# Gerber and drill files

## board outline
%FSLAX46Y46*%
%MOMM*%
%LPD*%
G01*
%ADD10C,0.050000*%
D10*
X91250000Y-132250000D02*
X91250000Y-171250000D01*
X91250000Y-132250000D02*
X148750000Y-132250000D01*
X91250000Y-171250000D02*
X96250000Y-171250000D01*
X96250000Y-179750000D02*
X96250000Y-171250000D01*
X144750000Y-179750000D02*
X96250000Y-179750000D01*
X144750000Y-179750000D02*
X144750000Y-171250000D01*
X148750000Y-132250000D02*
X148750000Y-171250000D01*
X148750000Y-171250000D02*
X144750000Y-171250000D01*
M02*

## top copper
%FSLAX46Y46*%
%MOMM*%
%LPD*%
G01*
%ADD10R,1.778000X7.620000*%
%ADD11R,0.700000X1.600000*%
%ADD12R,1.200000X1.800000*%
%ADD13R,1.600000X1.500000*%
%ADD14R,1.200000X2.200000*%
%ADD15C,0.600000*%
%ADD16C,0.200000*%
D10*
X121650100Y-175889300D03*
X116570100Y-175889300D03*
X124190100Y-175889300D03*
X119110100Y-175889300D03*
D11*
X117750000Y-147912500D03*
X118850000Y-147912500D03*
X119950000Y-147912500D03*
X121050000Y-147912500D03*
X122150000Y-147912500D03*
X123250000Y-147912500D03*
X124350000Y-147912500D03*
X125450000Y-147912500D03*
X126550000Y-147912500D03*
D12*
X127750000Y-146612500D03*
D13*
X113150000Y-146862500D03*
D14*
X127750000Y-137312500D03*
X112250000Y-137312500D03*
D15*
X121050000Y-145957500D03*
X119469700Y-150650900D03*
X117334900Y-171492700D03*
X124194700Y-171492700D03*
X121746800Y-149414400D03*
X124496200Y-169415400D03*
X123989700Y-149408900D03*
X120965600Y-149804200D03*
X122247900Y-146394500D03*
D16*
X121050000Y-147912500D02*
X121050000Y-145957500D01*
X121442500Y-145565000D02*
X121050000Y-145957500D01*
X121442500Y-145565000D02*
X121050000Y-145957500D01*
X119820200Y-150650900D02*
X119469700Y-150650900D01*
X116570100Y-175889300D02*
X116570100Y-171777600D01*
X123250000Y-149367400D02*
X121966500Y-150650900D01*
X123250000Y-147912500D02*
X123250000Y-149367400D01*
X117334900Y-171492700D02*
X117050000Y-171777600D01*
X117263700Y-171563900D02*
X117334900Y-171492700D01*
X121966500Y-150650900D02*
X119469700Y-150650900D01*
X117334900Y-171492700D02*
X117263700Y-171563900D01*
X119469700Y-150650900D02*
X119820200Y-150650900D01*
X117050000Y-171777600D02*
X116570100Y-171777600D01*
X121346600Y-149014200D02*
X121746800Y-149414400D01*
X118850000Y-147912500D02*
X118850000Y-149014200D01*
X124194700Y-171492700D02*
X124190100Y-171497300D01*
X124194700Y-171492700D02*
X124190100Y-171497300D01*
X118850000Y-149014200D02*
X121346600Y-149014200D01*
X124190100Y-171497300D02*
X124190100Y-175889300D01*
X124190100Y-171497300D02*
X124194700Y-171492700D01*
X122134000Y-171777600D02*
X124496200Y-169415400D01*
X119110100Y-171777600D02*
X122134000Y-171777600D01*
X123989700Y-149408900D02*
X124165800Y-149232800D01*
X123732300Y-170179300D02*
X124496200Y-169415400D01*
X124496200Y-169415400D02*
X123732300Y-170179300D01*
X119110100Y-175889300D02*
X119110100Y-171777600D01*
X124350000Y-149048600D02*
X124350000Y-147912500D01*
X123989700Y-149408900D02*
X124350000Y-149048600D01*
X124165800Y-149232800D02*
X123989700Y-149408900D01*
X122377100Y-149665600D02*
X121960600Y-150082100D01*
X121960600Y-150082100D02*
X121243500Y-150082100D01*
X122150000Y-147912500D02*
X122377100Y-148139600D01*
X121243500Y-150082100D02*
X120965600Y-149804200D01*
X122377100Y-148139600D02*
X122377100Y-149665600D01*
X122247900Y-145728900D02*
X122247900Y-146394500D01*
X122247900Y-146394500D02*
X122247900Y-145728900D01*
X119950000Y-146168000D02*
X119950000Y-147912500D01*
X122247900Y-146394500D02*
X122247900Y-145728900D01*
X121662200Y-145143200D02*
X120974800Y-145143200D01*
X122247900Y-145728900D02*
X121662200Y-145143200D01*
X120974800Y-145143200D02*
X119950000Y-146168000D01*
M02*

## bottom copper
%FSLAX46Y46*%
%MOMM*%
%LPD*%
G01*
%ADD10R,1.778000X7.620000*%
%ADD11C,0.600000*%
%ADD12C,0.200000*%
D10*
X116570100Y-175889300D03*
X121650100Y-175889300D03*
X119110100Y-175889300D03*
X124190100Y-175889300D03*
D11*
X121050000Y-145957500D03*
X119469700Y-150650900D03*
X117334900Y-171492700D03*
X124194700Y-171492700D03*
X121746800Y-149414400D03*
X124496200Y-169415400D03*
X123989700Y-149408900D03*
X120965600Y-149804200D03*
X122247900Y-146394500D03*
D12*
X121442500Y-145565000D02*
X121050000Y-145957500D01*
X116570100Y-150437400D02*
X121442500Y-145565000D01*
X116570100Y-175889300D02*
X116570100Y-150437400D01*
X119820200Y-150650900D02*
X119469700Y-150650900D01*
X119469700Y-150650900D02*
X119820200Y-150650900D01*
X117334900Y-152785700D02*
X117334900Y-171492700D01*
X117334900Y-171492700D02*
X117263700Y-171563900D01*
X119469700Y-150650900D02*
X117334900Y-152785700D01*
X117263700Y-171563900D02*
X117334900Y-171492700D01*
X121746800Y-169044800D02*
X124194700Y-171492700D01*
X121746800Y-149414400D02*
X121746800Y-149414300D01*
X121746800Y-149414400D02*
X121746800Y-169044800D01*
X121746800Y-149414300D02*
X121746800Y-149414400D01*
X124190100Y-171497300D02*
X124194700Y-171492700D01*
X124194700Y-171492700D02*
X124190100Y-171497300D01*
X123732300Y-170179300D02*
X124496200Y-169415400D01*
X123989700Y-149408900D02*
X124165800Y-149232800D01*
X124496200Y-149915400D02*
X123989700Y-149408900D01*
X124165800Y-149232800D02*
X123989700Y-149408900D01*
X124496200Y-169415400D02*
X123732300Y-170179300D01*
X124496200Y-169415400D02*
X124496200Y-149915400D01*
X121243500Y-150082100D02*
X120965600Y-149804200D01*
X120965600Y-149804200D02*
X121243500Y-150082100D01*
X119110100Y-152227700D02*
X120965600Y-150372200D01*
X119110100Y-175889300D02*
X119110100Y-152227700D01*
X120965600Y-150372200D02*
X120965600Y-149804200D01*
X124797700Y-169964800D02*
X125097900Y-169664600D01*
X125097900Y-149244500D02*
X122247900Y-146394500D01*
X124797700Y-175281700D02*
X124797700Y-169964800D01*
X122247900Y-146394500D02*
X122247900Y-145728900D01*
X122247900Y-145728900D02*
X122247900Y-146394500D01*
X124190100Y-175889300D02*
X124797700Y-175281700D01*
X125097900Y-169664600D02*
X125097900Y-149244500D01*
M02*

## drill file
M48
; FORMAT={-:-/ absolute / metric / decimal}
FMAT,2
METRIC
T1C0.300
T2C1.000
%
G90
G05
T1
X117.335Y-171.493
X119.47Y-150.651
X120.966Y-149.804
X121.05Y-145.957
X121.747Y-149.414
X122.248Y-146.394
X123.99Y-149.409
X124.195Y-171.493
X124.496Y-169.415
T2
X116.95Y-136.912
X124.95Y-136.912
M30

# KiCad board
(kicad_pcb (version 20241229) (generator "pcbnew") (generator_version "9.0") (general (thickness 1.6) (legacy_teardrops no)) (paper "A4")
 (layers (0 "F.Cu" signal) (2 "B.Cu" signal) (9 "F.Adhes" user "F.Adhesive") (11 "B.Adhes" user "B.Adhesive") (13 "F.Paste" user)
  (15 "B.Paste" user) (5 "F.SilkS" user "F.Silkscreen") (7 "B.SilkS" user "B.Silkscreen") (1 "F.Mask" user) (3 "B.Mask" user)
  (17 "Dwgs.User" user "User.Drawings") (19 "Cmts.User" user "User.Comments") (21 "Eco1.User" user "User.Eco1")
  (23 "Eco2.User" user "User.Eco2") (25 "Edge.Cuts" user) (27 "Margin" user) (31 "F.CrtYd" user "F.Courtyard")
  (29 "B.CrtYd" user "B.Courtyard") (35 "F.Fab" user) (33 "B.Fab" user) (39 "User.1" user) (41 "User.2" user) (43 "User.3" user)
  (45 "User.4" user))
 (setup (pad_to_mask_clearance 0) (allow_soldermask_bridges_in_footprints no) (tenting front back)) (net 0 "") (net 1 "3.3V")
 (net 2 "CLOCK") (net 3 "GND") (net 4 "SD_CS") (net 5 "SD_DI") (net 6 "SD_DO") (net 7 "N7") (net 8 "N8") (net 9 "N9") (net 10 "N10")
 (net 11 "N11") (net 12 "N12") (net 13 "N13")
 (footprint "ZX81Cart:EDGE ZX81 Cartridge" (layer "F.Cu") (at 119.7451 172.7143)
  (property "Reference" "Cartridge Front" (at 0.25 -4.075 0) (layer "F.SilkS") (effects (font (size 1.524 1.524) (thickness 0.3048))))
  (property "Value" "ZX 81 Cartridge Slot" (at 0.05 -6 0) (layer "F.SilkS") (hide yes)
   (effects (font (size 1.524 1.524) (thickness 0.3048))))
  (pad "3.3V" connect rect (at -3.175 3.175 180) (size 1.778 7.62) (layers "B.Cu" "B.Mask") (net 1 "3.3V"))
  (pad "A3" connect rect (at 1.905 3.175 180) (size 1.778 7.62) (layers "F.Cu" "F.Mask"))
  (pad "B3" connect rect (at 1.905 3.175 180) (size 1.778 7.62) (layers "B.Cu" "B.Mask"))
  (pad "CLOCK" connect rect (at -0.635 3.175 180) (size 1.778 7.62) (layers "B.Cu" "B.Mask") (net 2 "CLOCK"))
  (pad "GND" connect rect (at -3.175 3.175 180) (size 1.778 7.62) (layers "F.Cu" "F.Mask") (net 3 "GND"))
  (pad "SD_CS" connect rect (at 4.445 3.175 180) (size 1.778 7.62) (layers "F.Cu" "F.Mask") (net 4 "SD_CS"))
  (pad "SD_DI" connect rect (at -0.635 3.175 180) (size 1.778 7.62) (layers "F.Cu" "F.Mask") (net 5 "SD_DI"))
  (pad "SD_DO" connect rect (at 4.445 3.175 180) (size 1.778 7.62) (layers "B.Cu" "B.Mask") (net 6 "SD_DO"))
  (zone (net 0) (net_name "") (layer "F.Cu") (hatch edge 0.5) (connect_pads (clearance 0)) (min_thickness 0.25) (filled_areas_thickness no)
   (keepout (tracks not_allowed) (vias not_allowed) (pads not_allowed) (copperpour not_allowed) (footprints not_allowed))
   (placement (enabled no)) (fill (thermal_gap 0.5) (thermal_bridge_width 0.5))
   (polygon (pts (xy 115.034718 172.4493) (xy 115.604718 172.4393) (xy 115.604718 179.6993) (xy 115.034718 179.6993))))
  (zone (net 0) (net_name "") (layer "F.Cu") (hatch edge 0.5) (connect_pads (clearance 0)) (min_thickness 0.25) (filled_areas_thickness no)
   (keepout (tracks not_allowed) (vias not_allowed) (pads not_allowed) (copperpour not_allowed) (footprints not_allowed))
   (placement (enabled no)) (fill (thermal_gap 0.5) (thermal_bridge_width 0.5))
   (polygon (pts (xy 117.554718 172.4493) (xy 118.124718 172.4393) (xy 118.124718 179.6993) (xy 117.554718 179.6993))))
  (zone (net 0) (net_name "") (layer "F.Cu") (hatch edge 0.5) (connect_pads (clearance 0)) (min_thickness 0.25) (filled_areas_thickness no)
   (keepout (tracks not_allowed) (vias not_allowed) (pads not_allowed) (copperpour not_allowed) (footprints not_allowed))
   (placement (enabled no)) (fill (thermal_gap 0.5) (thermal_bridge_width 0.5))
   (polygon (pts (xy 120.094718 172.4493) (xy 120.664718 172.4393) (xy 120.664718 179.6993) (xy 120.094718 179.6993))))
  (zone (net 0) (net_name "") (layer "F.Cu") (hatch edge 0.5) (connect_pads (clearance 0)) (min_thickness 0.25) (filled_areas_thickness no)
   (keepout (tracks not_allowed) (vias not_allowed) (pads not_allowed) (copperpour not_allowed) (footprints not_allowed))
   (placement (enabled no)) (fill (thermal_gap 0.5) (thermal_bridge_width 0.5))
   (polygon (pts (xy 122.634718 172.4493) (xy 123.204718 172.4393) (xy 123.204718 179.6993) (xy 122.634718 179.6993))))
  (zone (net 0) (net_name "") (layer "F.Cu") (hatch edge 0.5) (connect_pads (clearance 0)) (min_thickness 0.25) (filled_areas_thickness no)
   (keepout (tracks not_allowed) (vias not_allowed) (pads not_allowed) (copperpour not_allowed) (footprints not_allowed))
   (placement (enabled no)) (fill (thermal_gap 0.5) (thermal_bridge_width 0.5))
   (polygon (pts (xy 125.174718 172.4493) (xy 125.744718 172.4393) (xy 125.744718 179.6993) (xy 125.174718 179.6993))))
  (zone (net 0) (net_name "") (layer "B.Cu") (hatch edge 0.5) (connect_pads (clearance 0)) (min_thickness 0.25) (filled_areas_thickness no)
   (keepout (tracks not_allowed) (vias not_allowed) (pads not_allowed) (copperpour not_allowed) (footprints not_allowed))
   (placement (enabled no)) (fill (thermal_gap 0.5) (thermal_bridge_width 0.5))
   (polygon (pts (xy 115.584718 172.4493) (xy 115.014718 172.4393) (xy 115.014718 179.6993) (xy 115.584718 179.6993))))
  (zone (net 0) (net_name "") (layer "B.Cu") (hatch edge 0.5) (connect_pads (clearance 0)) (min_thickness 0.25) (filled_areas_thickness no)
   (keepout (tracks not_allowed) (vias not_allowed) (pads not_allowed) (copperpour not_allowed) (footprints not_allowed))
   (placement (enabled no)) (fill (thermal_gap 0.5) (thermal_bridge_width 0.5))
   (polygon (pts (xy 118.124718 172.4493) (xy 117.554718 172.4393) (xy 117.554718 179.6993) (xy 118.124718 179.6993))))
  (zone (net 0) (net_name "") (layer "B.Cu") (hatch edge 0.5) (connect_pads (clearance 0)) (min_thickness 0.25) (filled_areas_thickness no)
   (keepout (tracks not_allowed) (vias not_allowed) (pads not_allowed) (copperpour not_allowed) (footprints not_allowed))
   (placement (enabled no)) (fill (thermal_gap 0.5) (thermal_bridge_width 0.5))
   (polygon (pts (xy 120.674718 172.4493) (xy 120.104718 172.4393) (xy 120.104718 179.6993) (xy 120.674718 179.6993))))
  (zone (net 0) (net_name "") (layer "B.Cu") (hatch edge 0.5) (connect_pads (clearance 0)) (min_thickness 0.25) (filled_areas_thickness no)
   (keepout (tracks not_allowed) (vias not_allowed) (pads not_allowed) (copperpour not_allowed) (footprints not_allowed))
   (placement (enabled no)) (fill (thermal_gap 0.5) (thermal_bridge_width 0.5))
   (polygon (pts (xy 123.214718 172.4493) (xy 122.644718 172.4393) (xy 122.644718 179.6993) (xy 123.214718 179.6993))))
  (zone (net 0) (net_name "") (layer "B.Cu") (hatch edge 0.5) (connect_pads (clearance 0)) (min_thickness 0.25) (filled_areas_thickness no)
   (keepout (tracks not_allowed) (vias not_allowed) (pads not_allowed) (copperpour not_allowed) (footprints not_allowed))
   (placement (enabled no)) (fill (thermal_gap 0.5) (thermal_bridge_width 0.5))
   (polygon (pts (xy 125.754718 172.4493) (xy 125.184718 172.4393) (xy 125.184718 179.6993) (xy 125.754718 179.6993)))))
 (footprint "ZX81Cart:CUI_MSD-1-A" (layer "F.Cu") (at 120 140.1625 180)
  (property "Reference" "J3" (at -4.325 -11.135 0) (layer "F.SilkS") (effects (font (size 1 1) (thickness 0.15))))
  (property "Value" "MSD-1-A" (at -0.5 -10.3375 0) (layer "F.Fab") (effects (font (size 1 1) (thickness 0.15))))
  (pad "" np_thru_hole circle (at -4.95 3.25 180) (size 1 1) (drill 1) (layers "*.Cu" "*.Mask"))
  (pad "" np_thru_hole circle (at 3.05 3.25 180) (size 1 1) (drill 1) (layers "*.Cu" "*.Mask"))
  (pad "1" smd rect (at 2.25 -7.75 180) (size 0.7 1.6) (layers "F.Cu" "F.Mask" "F.Paste") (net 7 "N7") (solder_mask_margin 0.102))
  (pad "2" smd rect (at 1.15 -7.75 180) (size 0.7 1.6) (layers "F.Cu" "F.Mask" "F.Paste") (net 4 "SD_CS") (solder_mask_margin 0.102))
  (pad "3" smd rect (at 0.05 -7.75 180) (size 0.7 1.6) (layers "F.Cu" "F.Mask" "F.Paste") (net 6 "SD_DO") (solder_mask_margin 0.102))
  (pad "4" smd rect (at -1.05 -7.75 180) (size 0.7 1.6) (layers "F.Cu" "F.Mask" "F.Paste") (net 1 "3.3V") (solder_mask_margin 0.102))
  (pad "5" smd rect (at -2.15 -7.75 180) (size 0.7 1.6) (layers "F.Cu" "F.Mask" "F.Paste") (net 2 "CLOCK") (solder_mask_margin 0.102))
  (pad "6" smd rect (at -3.25 -7.75 180) (size 0.7 1.6) (layers "F.Cu" "F.Mask" "F.Paste") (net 3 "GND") (solder_mask_margin 0.102))
  (pad "7" smd rect (at -4.35 -7.75 180) (size 0.7 1.6) (layers "F.Cu" "F.Mask" "F.Paste") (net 5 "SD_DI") (solder_mask_margin 0.102))
  (pad "8" smd rect (at -5.45 -7.75 180) (size 0.7 1.6) (layers "F.Cu" "F.Mask" "F.Paste") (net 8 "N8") (solder_mask_margin 0.102))
  (pad "CD" smd rect (at -6.55 -7.75 180) (size 0.7 1.6) (layers "F.Cu" "F.Mask" "F.Paste") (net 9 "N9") (solder_mask_margin 0.102))
  (pad "G1" smd rect (at -7.75 -6.45 180) (size 1.2 1.8) (layers "F.Cu" "F.Mask" "F.Paste") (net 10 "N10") (solder_mask_margin 0.102))
  (pad "G2" smd rect (at 6.85 -6.7 180) (size 1.6 1.5) (layers "F.Cu" "F.Mask" "F.Paste") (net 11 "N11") (solder_mask_margin 0.102))
  (pad "G3" smd rect (at -7.75 2.85 180) (size 1.2 2.2) (layers "F.Cu" "F.Mask" "F.Paste") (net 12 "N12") (solder_mask_margin 0.102))
  (pad "G4" smd rect (at 7.75 2.85 180) (size 1.2 2.2) (layers "F.Cu" "F.Mask" "F.Paste") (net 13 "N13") (solder_mask_margin 0.102)))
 (gr_line (start 91.25 132.25) (end 91.25 171.25) (stroke (width 0.05) (type default)) (layer "Edge.Cuts"))
 (gr_line (start 91.25 132.25) (end 148.75 132.25) (stroke (width 0.05) (type default)) (layer "Edge.Cuts"))
 (gr_line (start 91.25 171.25) (end 96.25 171.25) (stroke (width 0.05) (type default)) (layer "Edge.Cuts"))
 (gr_line (start 96.25 179.75) (end 96.25 171.25) (stroke (width 0.05) (type default)) (layer "Edge.Cuts"))
 (gr_line (start 144.75 179.75) (end 96.25 179.75) (stroke (width 0.05) (type solid)) (layer "Edge.Cuts"))
 (gr_line (start 144.75 179.75) (end 144.75 171.25) (stroke (width 0.05) (type default)) (layer "Edge.Cuts"))
 (gr_line (start 148.75 132.25) (end 148.75 171.25) (stroke (width 0.05) (type default)) (layer "Edge.Cuts"))
 (gr_line (start 148.75 171.25) (end 144.75 171.25) (stroke (width 0.05) (type default)) (layer "Edge.Cuts"))
 (segment (start 121.05 147.9125) (end 121.05 145.9575) (width 0.2) (layer "F.Cu") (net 1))
 (segment (start 121.4425 145.565) (end 121.05 145.9575) (width 0.2) (layer "F.Cu") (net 1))
 (segment (start 121.4425 145.565) (end 121.05 145.9575) (width 0.2) (layer "F.Cu") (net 1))
 (via (at 121.05 145.9575) (size 0.6) (drill 0.3) (layers "F.Cu" "B.Cu") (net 1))
 (segment (start 121.4425 145.565) (end 121.05 145.9575) (width 0.2) (layer "B.Cu") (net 1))
 (segment (start 116.5701 150.4374) (end 121.4425 145.565) (width 0.2) (layer "B.Cu") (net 1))
 (segment (start 116.5701 175.8893) (end 116.5701 150.4374) (width 0.2) (layer "B.Cu") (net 1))
 (segment (start 119.8202 150.6509) (end 119.4697 150.6509) (width 0.2) (layer "F.Cu") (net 3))
 (segment (start 116.5701 175.8893) (end 116.5701 171.7776) (width 0.2) (layer "F.Cu") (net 3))
 (segment (start 123.25 149.3674) (end 121.9665 150.6509) (width 0.2) (layer "F.Cu") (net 3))
 (segment (start 123.25 147.9125) (end 123.25 149.3674) (width 0.2) (layer "F.Cu") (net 3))
 (segment (start 117.3349 171.4927) (end 117.05 171.7776) (width 0.2) (layer "F.Cu") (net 3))
 (segment (start 117.2637 171.5639) (end 117.3349 171.4927) (width 0.2) (layer "F.Cu") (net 3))
 (segment (start 121.9665 150.6509) (end 119.4697 150.6509) (width 0.2) (layer "F.Cu") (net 3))
 (segment (start 117.3349 171.4927) (end 117.2637 171.5639) (width 0.2) (layer "F.Cu") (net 3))
 (segment (start 119.4697 150.6509) (end 119.8202 150.6509) (width 0.2) (layer "F.Cu") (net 3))
 (segment (start 117.05 171.7776) (end 116.5701 171.7776) (width 0.2) (layer "F.Cu") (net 3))
 (via (at 119.4697 150.6509) (size 0.6) (drill 0.3) (layers "F.Cu" "B.Cu") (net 3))
 (via (at 117.3349 171.4927) (size 0.6) (drill 0.3) (layers "F.Cu" "B.Cu") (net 3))
 (segment (start 119.8202 150.6509) (end 119.4697 150.6509) (width 0.2) (layer "B.Cu") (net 3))
 (segment (start 119.4697 150.6509) (end 119.8202 150.6509) (width 0.2) (layer "B.Cu") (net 3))
 (segment (start 117.3349 152.7857) (end 117.3349 171.4927) (width 0.2) (layer "B.Cu") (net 3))
 (segment (start 117.3349 171.4927) (end 117.2637 171.5639) (width 0.2) (layer "B.Cu") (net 3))
 (segment (start 119.4697 150.6509) (end 117.3349 152.7857) (width 0.2) (layer "B.Cu") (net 3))
 (segment (start 117.2637 171.5639) (end 117.3349 171.4927) (width 0.2) (layer "B.Cu") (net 3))
 (segment (start 121.3466 149.0142) (end 121.7468 149.4144) (width 0.2) (layer "F.Cu") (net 4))
 (segment (start 118.85 147.9125) (end 118.85 149.0142) (width 0.2) (layer "F.Cu") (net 4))
 (segment (start 124.1947 171.4927) (end 124.1901 171.4973) (width 0.2) (layer "F.Cu") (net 4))
 (segment (start 124.1947 171.4927) (end 124.1901 171.4973) (width 0.2) (layer "F.Cu") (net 4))
 (segment (start 118.85 149.0142) (end 121.3466 149.0142) (width 0.2) (layer "F.Cu") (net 4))
 (segment (start 124.1901 171.4973) (end 124.1901 175.8893) (width 0.2) (layer "F.Cu") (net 4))
 (segment (start 124.1901 171.4973) (end 124.1947 171.4927) (width 0.2) (layer "F.Cu") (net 4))
 (via (at 124.1947 171.4927) (size 0.6) (drill 0.3) (layers "F.Cu" "B.Cu") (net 4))
 (via (at 121.7468 149.4144) (size 0.6) (drill 0.3) (layers "F.Cu" "B.Cu") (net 4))
 (segment (start 121.7468 169.0448) (end 124.1947 171.4927) (width 0.2) (layer "B.Cu") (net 4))
 (segment (start 121.7468 149.4144) (end 121.7468 149.4143) (width 0.2) (layer "B.Cu") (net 4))
 (segment (start 121.7468 149.4144) (end 121.7468 169.0448) (width 0.2) (layer "B.Cu") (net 4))
 (segment (start 121.7468 149.4143) (end 121.7468 149.4144) (width 0.2) (layer "B.Cu") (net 4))
 (segment (start 124.1901 171.4973) (end 124.1947 171.4927) (width 0.2) (layer "B.Cu") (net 4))
 (segment (start 124.1947 171.4927) (end 124.1901 171.4973) (width 0.2) (layer "B.Cu") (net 4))
 (segment (start 122.134 171.7776) (end 124.4962 169.4154) (width 0.2) (layer "F.Cu") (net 5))
 (segment (start 119.1101 171.7776) (end 122.134 171.7776) (width 0.2) (layer "F.Cu") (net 5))
 (segment (start 123.9897 149.4089) (end 124.1658 149.2328) (width 0.2) (layer "F.Cu") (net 5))
 (segment (start 123.7323 170.1793) (end 124.4962 169.4154) (width 0.2) (layer "F.Cu") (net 5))
 (segment (start 124.4962 169.4154) (end 123.7323 170.1793) (width 0.2) (layer "F.Cu") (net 5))
 (segment (start 119.1101 175.8893) (end 119.1101 171.7776) (width 0.2) (layer "F.Cu") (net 5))
 (segment (start 124.35 149.0486) (end 124.35 147.9125) (width 0.2) (layer "F.Cu") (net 5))
 (segment (start 123.9897 149.4089) (end 124.35 149.0486) (width 0.2) (layer "F.Cu") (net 5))
 (segment (start 124.1658 149.2328) (end 123.9897 149.4089) (width 0.2) (layer "F.Cu") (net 5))
 (via (at 124.4962 169.4154) (size 0.6) (drill 0.3) (layers "F.Cu" "B.Cu") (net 5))
 (via (at 123.9897 149.4089) (size 0.6) (drill 0.3) (layers "F.Cu" "B.Cu") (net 5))
 (segment (start 123.7323 170.1793) (end 124.4962 169.4154) (width 0.2) (layer "B.Cu") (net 5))
 (segment (start 123.9897 149.4089) (end 124.1658 149.2328) (width 0.2) (layer "B.Cu") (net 5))
 (segment (start 124.4962 149.9154) (end 123.9897 149.4089) (width 0.2) (layer "B.Cu") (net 5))
 (segment (start 124.1658 149.2328) (end 123.9897 149.4089) (width 0.2) (layer "B.Cu") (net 5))
 (segment (start 124.4962 169.4154) (end 123.7323 170.1793) (width 0.2) (layer "B.Cu") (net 5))
 (segment (start 124.4962 169.4154) (end 124.4962 149.9154) (width 0.2) (layer "B.Cu") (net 5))
 (segment (start 122.3771 149.6656) (end 121.9606 150.0821) (width 0.2) (layer "F.Cu") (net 2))
 (segment (start 121.9606 150.0821) (end 121.2435 150.0821) (width 0.2) (layer "F.Cu") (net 2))
 (segment (start 122.15 147.9125) (end 122.3771 148.1396) (width 0.2) (layer "F.Cu") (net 2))
 (segment (start 121.2435 150.0821) (end 120.9656 149.8042) (width 0.2) (layer "F.Cu") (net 2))
 (segment (start 122.3771 148.1396) (end 122.3771 149.6656) (width 0.2) (layer "F.Cu") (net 2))
 (via (at 120.9656 149.8042) (size 0.6) (drill 0.3) (layers "F.Cu" "B.Cu") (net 2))
 (segment (start 121.2435 150.0821) (end 120.9656 149.8042) (width 0.2) (layer "B.Cu") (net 2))
 (segment (start 120.9656 149.8042) (end 121.2435 150.0821) (width 0.2) (layer "B.Cu") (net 2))
 (segment (start 119.1101 152.2277) (end 120.9656 150.3722) (width 0.2) (layer "B.Cu") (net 2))
 (segment (start 119.1101 175.8893) (end 119.1101 152.2277) (width 0.2) (layer "B.Cu") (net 2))
 (segment (start 120.9656 150.3722) (end 120.9656 149.8042) (width 0.2) (layer "B.Cu") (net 2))
 (segment (start 122.2479 145.7289) (end 122.2479 146.3945) (width 0.2) (layer "F.Cu") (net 6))
 (segment (start 122.2479 146.3945) (end 122.2479 145.7289) (width 0.2) (layer "F.Cu") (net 6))
 (segment (start 119.95 146.168) (end 119.95 147.9125) (width 0.2) (layer "F.Cu") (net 6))
 (segment (start 122.2479 146.3945) (end 122.2479 145.7289) (width 0.2) (layer "F.Cu") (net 6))
 (segment (start 121.6622 145.1432) (end 120.9748 145.1432) (width 0.2) (layer "F.Cu") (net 6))
 (segment (start 122.2479 145.7289) (end 121.6622 145.1432) (width 0.2) (layer "F.Cu") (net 6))
 (segment (start 120.9748 145.1432) (end 119.95 146.168) (width 0.2) (layer "F.Cu") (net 6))
 (via (at 122.2479 146.3945) (size 0.6) (drill 0.3) (layers "F.Cu" "B.Cu") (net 6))
 (segment (start 124.7977 169.9648) (end 125.0979 169.6646) (width 0.2) (layer "B.Cu") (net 6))
 (segment (start 125.0979 149.2445) (end 122.2479 146.3945) (width 0.2) (layer "B.Cu") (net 6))
 (segment (start 124.7977 175.2817) (end 124.7977 169.9648) (width 0.2) (layer "B.Cu") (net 6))
 (segment (start 122.2479 146.3945) (end 122.2479 145.7289) (width 0.2) (layer "B.Cu") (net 6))
 (segment (start 122.2479 145.7289) (end 122.2479 146.3945) (width 0.2) (layer "B.Cu") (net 6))
 (segment (start 124.1901 175.8893) (end 124.7977 175.2817) (width 0.2) (layer "B.Cu") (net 6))
 (segment (start 125.0979 169.6646) (end 125.0979 149.2445) (width 0.2) (layer "B.Cu") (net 6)))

